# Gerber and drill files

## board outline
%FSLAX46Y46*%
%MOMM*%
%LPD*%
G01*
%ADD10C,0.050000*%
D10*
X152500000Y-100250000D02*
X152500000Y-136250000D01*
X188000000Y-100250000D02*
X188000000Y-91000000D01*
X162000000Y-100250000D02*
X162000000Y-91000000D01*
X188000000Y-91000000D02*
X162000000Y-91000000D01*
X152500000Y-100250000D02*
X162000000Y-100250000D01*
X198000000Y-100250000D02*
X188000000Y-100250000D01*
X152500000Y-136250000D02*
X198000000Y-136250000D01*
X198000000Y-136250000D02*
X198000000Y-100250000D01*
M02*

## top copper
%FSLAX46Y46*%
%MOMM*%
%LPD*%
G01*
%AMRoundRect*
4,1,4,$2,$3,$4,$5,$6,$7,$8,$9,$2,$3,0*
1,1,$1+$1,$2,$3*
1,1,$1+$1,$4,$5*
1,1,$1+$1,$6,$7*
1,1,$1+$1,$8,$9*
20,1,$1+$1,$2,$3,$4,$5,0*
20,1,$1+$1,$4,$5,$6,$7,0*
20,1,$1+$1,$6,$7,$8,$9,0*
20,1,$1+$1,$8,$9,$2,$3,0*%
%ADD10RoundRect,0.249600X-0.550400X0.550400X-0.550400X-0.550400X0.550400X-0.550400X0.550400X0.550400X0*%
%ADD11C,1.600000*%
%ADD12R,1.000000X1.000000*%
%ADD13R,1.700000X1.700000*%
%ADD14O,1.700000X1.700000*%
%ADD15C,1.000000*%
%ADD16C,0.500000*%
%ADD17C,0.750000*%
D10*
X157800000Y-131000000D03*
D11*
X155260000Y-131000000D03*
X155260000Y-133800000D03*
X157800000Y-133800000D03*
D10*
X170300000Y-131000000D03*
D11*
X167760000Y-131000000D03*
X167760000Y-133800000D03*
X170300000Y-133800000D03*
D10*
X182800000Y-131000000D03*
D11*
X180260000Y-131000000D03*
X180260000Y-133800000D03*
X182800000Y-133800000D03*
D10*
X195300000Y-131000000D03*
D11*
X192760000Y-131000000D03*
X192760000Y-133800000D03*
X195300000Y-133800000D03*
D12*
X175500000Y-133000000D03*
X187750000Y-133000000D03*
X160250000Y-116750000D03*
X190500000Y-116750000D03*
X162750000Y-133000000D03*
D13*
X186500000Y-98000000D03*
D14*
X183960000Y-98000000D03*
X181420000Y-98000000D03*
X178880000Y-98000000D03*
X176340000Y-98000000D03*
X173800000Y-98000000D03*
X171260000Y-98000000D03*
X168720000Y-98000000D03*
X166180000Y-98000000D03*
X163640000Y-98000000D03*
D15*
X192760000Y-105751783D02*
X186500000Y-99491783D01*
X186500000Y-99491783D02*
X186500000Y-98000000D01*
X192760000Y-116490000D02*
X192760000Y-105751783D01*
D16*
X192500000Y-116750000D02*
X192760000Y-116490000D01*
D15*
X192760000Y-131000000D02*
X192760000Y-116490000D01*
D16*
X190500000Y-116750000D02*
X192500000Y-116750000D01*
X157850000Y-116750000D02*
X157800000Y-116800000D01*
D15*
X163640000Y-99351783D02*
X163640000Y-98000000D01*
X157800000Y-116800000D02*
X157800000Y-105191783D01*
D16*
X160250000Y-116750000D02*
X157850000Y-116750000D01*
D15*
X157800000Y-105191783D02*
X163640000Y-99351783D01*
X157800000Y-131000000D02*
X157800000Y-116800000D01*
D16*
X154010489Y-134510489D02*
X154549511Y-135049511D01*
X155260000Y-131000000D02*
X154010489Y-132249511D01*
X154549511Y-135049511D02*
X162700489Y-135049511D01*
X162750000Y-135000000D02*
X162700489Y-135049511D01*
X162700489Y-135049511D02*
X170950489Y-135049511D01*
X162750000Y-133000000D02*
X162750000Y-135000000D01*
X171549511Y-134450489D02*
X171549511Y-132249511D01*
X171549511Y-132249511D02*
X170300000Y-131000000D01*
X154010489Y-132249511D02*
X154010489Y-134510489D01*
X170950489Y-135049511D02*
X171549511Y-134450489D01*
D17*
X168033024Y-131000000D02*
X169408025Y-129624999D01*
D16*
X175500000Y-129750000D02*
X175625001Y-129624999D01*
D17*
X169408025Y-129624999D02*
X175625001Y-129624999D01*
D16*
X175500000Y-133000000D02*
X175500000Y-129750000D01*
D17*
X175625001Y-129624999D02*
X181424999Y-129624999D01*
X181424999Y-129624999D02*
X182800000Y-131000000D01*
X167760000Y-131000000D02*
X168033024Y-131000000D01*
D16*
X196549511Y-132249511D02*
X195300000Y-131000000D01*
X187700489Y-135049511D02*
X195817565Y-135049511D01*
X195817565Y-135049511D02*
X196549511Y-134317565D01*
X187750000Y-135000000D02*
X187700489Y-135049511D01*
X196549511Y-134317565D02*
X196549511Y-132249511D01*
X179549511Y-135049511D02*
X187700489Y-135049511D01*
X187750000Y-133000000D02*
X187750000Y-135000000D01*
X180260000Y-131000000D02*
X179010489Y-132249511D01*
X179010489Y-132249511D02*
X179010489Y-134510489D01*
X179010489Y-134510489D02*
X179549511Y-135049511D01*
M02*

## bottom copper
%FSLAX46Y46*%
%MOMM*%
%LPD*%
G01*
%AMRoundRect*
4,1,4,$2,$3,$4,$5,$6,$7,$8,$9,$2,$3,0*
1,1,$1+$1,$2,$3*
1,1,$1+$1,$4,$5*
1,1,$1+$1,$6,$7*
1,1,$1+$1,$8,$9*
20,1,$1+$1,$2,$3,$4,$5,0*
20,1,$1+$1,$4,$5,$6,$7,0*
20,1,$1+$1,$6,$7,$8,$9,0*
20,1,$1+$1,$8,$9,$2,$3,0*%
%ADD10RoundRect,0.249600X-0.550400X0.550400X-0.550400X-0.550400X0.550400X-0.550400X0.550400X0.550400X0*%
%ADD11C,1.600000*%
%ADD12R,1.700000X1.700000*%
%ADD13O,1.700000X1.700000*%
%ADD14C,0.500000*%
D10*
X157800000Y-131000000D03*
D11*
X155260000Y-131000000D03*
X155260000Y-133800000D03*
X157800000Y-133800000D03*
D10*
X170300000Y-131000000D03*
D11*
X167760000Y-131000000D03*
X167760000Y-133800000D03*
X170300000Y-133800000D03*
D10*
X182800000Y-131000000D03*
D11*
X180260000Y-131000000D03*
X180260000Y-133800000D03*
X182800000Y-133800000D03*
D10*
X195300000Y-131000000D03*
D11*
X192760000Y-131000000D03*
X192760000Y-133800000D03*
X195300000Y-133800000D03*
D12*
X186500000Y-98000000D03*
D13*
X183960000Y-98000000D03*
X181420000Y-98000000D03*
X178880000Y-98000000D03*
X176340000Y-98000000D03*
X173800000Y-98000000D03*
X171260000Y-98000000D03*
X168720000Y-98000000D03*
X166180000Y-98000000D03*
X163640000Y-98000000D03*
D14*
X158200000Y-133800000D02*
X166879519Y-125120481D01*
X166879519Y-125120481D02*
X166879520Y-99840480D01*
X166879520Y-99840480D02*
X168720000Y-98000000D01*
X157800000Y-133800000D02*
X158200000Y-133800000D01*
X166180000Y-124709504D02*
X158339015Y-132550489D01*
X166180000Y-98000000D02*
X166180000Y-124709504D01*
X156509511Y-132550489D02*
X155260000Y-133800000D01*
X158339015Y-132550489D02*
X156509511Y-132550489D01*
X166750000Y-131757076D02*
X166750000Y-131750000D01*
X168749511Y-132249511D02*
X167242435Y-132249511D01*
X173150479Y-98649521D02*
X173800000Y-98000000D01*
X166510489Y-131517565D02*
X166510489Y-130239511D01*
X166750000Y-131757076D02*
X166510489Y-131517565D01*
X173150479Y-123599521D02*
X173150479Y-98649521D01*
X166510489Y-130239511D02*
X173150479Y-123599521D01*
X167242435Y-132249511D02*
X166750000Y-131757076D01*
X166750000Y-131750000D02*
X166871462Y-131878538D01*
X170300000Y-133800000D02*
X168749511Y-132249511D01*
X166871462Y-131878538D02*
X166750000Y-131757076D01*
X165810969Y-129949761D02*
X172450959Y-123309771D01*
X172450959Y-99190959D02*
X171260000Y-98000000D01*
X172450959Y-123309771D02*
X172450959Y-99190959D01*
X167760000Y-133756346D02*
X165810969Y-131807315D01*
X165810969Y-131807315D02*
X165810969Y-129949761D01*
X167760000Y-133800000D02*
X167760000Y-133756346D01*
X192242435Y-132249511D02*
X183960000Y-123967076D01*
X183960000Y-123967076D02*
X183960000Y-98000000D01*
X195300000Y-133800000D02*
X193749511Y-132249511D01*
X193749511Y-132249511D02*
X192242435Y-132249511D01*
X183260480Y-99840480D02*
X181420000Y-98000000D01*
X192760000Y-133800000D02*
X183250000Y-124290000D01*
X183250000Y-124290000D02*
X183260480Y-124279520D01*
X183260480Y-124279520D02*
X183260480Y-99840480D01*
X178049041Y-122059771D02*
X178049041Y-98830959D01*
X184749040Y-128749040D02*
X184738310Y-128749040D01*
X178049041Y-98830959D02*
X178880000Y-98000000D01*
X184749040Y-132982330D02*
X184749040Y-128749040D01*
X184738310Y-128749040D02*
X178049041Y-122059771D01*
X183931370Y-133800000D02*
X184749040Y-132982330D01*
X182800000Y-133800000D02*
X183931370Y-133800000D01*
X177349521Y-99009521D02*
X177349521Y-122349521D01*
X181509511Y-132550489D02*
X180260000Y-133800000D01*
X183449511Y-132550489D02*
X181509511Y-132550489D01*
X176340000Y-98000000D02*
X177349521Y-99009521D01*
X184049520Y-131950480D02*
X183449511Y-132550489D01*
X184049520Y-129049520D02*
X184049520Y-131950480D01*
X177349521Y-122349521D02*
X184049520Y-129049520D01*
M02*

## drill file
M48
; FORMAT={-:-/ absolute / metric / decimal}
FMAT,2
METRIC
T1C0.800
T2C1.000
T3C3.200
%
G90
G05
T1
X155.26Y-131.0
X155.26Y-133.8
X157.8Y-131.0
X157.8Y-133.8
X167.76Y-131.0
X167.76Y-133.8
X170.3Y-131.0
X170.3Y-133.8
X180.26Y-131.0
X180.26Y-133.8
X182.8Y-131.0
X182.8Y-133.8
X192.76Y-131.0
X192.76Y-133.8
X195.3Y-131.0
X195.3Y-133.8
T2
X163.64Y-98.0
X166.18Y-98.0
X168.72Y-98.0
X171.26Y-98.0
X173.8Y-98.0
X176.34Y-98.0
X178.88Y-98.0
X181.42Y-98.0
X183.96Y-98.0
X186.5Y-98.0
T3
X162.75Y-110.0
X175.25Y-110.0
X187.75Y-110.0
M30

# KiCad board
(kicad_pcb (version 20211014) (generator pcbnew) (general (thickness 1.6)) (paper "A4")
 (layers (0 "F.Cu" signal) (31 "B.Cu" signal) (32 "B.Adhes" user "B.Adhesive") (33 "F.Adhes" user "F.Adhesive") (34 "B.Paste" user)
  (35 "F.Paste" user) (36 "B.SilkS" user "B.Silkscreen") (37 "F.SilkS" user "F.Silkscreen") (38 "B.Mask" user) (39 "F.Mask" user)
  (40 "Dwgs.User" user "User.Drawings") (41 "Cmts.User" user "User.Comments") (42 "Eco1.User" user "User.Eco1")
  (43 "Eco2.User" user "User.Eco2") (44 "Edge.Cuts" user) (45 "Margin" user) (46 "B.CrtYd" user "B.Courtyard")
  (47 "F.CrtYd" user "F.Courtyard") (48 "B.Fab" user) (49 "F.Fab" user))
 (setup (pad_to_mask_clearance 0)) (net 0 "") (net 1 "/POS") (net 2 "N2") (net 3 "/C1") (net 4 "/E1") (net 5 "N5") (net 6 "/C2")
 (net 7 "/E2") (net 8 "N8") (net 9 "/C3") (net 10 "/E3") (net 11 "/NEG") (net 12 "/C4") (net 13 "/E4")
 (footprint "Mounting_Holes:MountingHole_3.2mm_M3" (layer "F.Cu") (at 162.75 110)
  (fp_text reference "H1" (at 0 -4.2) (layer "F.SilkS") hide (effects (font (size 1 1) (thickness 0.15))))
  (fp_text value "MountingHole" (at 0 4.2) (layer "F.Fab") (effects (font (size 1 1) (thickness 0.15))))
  (pad "" np_thru_hole circle locked (at 0 0) (size 3.2 3.2) (drill 3.2) (layers *.Cu *.Mask)))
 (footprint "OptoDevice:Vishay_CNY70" (layer "F.Cu") (at 157.8 131 -90)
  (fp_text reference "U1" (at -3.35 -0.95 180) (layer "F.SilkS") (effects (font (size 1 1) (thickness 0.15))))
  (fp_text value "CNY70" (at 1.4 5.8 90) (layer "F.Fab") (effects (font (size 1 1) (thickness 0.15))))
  (pad "1" thru_hole roundrect (at 0 0 270) (size 1.6 1.6) (drill 0.8) (layers *.Cu *.Mask) (roundrect_rratio 0.156) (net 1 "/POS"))
  (pad "2" thru_hole circle (at 0 2.54 270) (size 1.6 1.6) (drill 0.8) (layers *.Cu *.Mask) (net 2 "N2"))
  (pad "3" thru_hole circle (at 2.8 2.54 270) (size 1.6 1.6) (drill 0.8) (layers *.Cu *.Mask) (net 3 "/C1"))
  (pad "4" thru_hole circle (at 2.8 0 270) (size 1.6 1.6) (drill 0.8) (layers *.Cu *.Mask) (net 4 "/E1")))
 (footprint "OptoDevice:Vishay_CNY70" (layer "F.Cu") (at 170.3 131 -90)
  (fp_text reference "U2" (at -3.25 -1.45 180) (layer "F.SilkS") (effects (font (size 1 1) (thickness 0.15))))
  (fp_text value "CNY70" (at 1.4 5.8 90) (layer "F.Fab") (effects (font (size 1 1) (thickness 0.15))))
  (pad "1" thru_hole roundrect (at 0 0 270) (size 1.6 1.6) (drill 0.8) (layers *.Cu *.Mask) (roundrect_rratio 0.156) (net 2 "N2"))
  (pad "2" thru_hole circle (at 0 2.54 270) (size 1.6 1.6) (drill 0.8) (layers *.Cu *.Mask) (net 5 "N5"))
  (pad "3" thru_hole circle (at 2.8 2.54 270) (size 1.6 1.6) (drill 0.8) (layers *.Cu *.Mask) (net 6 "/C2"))
  (pad "4" thru_hole circle (at 2.8 0 270) (size 1.6 1.6) (drill 0.8) (layers *.Cu *.Mask) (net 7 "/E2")))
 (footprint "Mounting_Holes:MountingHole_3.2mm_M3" (layer "F.Cu") (at 175.25 110)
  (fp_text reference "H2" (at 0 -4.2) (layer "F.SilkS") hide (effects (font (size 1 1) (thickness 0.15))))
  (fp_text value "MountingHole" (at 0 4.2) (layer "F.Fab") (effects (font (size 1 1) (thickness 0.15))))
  (pad "" np_thru_hole circle locked (at 0 0) (size 3.2 3.2) (drill 3.2) (layers *.Cu *.Mask)))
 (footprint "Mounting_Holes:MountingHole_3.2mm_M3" (layer "F.Cu") (at 187.75 110)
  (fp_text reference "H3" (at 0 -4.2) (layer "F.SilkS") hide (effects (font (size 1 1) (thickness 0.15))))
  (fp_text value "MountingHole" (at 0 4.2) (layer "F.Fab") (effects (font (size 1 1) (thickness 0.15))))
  (pad "" np_thru_hole circle locked (at 0 0) (size 3.2 3.2) (drill 3.2) (layers *.Cu *.Mask)))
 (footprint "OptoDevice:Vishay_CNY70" (layer "F.Cu") (at 182.8 131 -90)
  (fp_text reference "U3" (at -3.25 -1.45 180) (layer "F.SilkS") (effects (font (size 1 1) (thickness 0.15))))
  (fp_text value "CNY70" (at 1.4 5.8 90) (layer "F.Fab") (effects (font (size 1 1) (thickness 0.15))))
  (pad "1" thru_hole roundrect (at 0 0 270) (size 1.6 1.6) (drill 0.8) (layers *.Cu *.Mask) (roundrect_rratio 0.156) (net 5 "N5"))
  (pad "2" thru_hole circle (at 0 2.54 270) (size 1.6 1.6) (drill 0.8) (layers *.Cu *.Mask) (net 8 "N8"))
  (pad "3" thru_hole circle (at 2.8 2.54 270) (size 1.6 1.6) (drill 0.8) (layers *.Cu *.Mask) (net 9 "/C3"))
  (pad "4" thru_hole circle (at 2.8 0 270) (size 1.6 1.6) (drill 0.8) (layers *.Cu *.Mask) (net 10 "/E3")))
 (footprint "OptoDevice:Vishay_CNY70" (layer "F.Cu") (at 195.3 131 -90)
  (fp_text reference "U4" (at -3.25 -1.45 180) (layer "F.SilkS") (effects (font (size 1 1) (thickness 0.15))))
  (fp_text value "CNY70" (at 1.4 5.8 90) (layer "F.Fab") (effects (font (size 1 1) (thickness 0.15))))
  (pad "1" thru_hole roundrect (at 0 0 270) (size 1.6 1.6) (drill 0.8) (layers *.Cu *.Mask) (roundrect_rratio 0.156) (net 8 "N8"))
  (pad "2" thru_hole circle (at 0 2.54 270) (size 1.6 1.6) (drill 0.8) (layers *.Cu *.Mask) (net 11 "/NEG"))
  (pad "3" thru_hole circle (at 2.8 2.54 270) (size 1.6 1.6) (drill 0.8) (layers *.Cu *.Mask) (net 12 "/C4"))
  (pad "4" thru_hole circle (at 2.8 0 270) (size 1.6 1.6) (drill 0.8) (layers *.Cu *.Mask) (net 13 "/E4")))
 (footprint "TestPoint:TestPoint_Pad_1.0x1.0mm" (layer "F.Cu") (at 175.5 133)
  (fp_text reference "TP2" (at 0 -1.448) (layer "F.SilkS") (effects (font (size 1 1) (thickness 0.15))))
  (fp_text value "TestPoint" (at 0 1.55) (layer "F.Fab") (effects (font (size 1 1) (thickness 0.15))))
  (pad "1" smd rect locked (at 0 0) (size 1 1) (layers "F.Cu" "F.Mask") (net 5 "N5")))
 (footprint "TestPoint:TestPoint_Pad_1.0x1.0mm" (layer "F.Cu") (at 187.75 133)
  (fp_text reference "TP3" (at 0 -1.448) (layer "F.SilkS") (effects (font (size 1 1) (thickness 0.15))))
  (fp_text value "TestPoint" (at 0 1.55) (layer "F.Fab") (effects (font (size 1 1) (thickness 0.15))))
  (pad "1" smd rect locked (at 0 0) (size 1 1) (layers "F.Cu" "F.Mask") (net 8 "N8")))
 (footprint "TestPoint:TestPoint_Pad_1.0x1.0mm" (layer "F.Cu") (at 160.25 116.75)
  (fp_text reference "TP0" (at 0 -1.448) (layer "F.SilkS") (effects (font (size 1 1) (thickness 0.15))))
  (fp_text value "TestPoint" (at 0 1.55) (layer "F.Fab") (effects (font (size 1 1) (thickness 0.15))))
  (pad "1" smd rect locked (at 0 0) (size 1 1) (layers "F.Cu" "F.Mask") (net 1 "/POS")))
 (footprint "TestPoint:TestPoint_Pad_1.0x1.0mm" (layer "F.Cu") (at 190.5 116.75)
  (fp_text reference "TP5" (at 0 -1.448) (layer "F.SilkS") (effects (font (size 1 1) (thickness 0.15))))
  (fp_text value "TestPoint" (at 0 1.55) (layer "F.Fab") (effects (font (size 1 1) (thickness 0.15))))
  (pad "1" smd rect locked (at 0 0) (size 1 1) (layers "F.Cu" "F.Mask") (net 11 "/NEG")))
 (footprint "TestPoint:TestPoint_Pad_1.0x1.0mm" (layer "F.Cu") (at 162.75 133)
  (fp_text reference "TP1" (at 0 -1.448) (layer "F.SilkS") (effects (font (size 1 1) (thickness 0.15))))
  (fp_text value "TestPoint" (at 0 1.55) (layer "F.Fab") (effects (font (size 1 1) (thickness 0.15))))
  (pad "1" smd rect locked (at 0 0) (size 1 1) (layers "F.Cu" "F.Mask") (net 2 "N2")))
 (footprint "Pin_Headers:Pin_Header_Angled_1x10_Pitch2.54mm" (layer "B.Cu") (at 186.5 98 90)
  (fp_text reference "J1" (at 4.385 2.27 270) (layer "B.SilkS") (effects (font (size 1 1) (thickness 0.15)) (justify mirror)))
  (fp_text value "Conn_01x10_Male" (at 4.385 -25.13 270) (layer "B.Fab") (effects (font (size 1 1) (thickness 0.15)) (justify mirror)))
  (pad "1" thru_hole rect (at 0 0 90) (size 1.7 1.7) (drill 1) (layers *.Cu *.Mask) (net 11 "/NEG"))
  (pad "2" thru_hole oval (at 0 -2.54 90) (size 1.7 1.7) (drill 1) (layers *.Cu *.Mask) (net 13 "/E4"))
  (pad "3" thru_hole oval (at 0 -5.08 90) (size 1.7 1.7) (drill 1) (layers *.Cu *.Mask) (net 12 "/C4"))
  (pad "4" thru_hole oval (at 0 -7.62 90) (size 1.7 1.7) (drill 1) (layers *.Cu *.Mask) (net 10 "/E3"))
  (pad "5" thru_hole oval (at 0 -10.16 90) (size 1.7 1.7) (drill 1) (layers *.Cu *.Mask) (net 9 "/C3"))
  (pad "6" thru_hole oval (at 0 -12.7 90) (size 1.7 1.7) (drill 1) (layers *.Cu *.Mask) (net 7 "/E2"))
  (pad "7" thru_hole oval (at 0 -15.24 90) (size 1.7 1.7) (drill 1) (layers *.Cu *.Mask) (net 6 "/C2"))
  (pad "8" thru_hole oval (at 0 -17.78 90) (size 1.7 1.7) (drill 1) (layers *.Cu *.Mask) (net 4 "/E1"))
  (pad "9" thru_hole oval (at 0 -20.32 90) (size 1.7 1.7) (drill 1) (layers *.Cu *.Mask) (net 3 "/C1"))
  (pad "10" thru_hole oval (at 0 -22.86 90) (size 1.7 1.7) (drill 1) (layers *.Cu *.Mask) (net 1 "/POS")))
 (gr_line (start 152.5 100.25) (end 152.5 136.25) (layer "Edge.Cuts") (width 0.05))
 (gr_line (start 188 100.25) (end 188 91) (layer "Edge.Cuts") (width 0.05))
 (gr_line (start 162 100.25) (end 162 91) (layer "Edge.Cuts") (width 0.05))
 (gr_line (start 188 91) (end 162 91) (layer "Edge.Cuts") (width 0.05))
 (gr_line (start 152.5 100.25) (end 162 100.25) (layer "Edge.Cuts") (width 0.05))
 (gr_line (start 198 100.25) (end 188 100.25) (layer "Edge.Cuts") (width 0.05))
 (gr_line (start 152.5 136.25) (end 198 136.25) (layer "Edge.Cuts") (width 0.05))
 (gr_line (start 198 136.25) (end 198 100.25) (layer "Edge.Cuts") (width 0.05))
 (segment (start 192.76 105.751783) (end 186.5 99.491783) (width 1) (layer "F.Cu") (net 11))
 (segment (start 186.5 99.491783) (end 186.5 98) (width 1) (layer "F.Cu") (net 11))
 (segment (start 192.76 116.49) (end 192.76 105.751783) (width 1) (layer "F.Cu") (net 11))
 (segment (start 192.5 116.75) (end 192.76 116.49) (width 0.5) (layer "F.Cu") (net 11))
 (segment (start 192.76 131) (end 192.76 116.49) (width 1) (layer "F.Cu") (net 11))
 (segment (start 190.5 116.75) (end 192.5 116.75) (width 0.5) (layer "F.Cu") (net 11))
 (segment (start 158.2 133.8) (end 166.879519 125.120481) (width 0.5) (layer "B.Cu") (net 4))
 (segment (start 166.879519 125.120481) (end 166.87952 99.84048) (width 0.5) (layer "B.Cu") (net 4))
 (segment (start 166.87952 99.84048) (end 168.72 98) (width 0.5) (layer "B.Cu") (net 4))
 (segment (start 157.8 133.8) (end 158.2 133.8) (width 0.5) (layer "B.Cu") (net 4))
 (segment (start 166.18 124.709504) (end 158.339015 132.550489) (width 0.5) (layer "B.Cu") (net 3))
 (segment (start 166.18 98) (end 166.18 124.709504) (width 0.5) (layer "B.Cu") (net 3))
 (segment (start 156.509511 132.550489) (end 155.26 133.8) (width 0.5) (layer "B.Cu") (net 3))
 (segment (start 158.339015 132.550489) (end 156.509511 132.550489) (width 0.5) (layer "B.Cu") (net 3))
 (segment (start 157.85 116.75) (end 157.8 116.8) (width 0.5) (layer "F.Cu") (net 1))
 (segment (start 163.64 99.351783) (end 163.64 98) (width 1) (layer "F.Cu") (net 1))
 (segment (start 157.8 116.8) (end 157.8 105.191783) (width 1) (layer "F.Cu") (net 1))
 (segment (start 160.25 116.75) (end 157.85 116.75) (width 0.5) (layer "F.Cu") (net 1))
 (segment (start 157.8 105.191783) (end 163.64 99.351783) (width 1) (layer "F.Cu") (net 1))
 (segment (start 157.8 131) (end 157.8 116.8) (width 1) (layer "F.Cu") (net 1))
 (segment (start 154.010489 134.510489) (end 154.549511 135.049511) (width 0.5) (layer "F.Cu") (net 2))
 (segment (start 155.26 131) (end 154.010489 132.249511) (width 0.5) (layer "F.Cu") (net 2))
 (segment (start 154.549511 135.049511) (end 162.700489 135.049511) (width 0.5) (layer "F.Cu") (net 2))
 (segment (start 162.75 135) (end 162.700489 135.049511) (width 0.5) (layer "F.Cu") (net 2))
 (segment (start 162.700489 135.049511) (end 170.950489 135.049511) (width 0.5) (layer "F.Cu") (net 2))
 (segment (start 162.75 133) (end 162.75 135) (width 0.5) (layer "F.Cu") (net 2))
 (segment (start 171.549511 134.450489) (end 171.549511 132.249511) (width 0.5) (layer "F.Cu") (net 2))
 (segment (start 171.549511 132.249511) (end 170.3 131) (width 0.5) (layer "F.Cu") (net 2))
 (segment (start 154.010489 132.249511) (end 154.010489 134.510489) (width 0.5) (layer "F.Cu") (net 2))
 (segment (start 170.950489 135.049511) (end 171.549511 134.450489) (width 0.5) (layer "F.Cu") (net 2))
 (segment (start 166.75 131.757076) (end 166.75 131.75) (width 0.5) (layer "B.Cu") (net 7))
 (segment (start 168.749511 132.249511) (end 167.242435 132.249511) (width 0.5) (layer "B.Cu") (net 7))
 (segment (start 173.150479 98.649521) (end 173.8 98) (width 0.5) (layer "B.Cu") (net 7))
 (segment (start 166.510489 131.517565) (end 166.510489 130.239511) (width 0.5) (layer "B.Cu") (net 7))
 (segment (start 166.75 131.757076) (end 166.510489 131.517565) (width 0.5) (layer "B.Cu") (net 7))
 (segment (start 173.150479 123.599521) (end 173.150479 98.649521) (width 0.5) (layer "B.Cu") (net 7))
 (segment (start 166.510489 130.239511) (end 173.150479 123.599521) (width 0.5) (layer "B.Cu") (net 7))
 (segment (start 167.242435 132.249511) (end 166.75 131.757076) (width 0.5) (layer "B.Cu") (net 7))
 (segment (start 166.75 131.75) (end 166.871462 131.878538) (width 0.5) (layer "B.Cu") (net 7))
 (segment (start 170.3 133.8) (end 168.749511 132.249511) (width 0.5) (layer "B.Cu") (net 7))
 (segment (start 166.871462 131.878538) (end 166.75 131.757076) (width 0.5) (layer "B.Cu") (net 7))
 (segment (start 165.810969 129.949761) (end 172.450959 123.309771) (width 0.5) (layer "B.Cu") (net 6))
 (segment (start 172.450959 99.190959) (end 171.26 98) (width 0.5) (layer "B.Cu") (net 6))
 (segment (start 172.450959 123.309771) (end 172.450959 99.190959) (width 0.5) (layer "B.Cu") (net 6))
 (segment (start 167.76 133.756346) (end 165.810969 131.807315) (width 0.5) (layer "B.Cu") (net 6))
 (segment (start 165.810969 131.807315) (end 165.810969 129.949761) (width 0.5) (layer "B.Cu") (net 6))
 (segment (start 167.76 133.8) (end 167.76 133.756346) (width 0.5) (layer "B.Cu") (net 6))
 (segment (start 192.242435 132.249511) (end 183.96 123.967076) (width 0.5) (layer "B.Cu") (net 13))
 (segment (start 183.96 123.967076) (end 183.96 98) (width 0.5) (layer "B.Cu") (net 13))
 (segment (start 195.3 133.8) (end 193.749511 132.249511) (width 0.5) (layer "B.Cu") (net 13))
 (segment (start 193.749511 132.249511) (end 192.242435 132.249511) (width 0.5) (layer "B.Cu") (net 13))
 (segment (start 183.26048 99.84048) (end 181.42 98) (width 0.5) (layer "B.Cu") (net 12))
 (segment (start 192.76 133.8) (end 183.25 124.29) (width 0.5) (layer "B.Cu") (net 12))
 (segment (start 183.25 124.29) (end 183.26048 124.27952) (width 0.5) (layer "B.Cu") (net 12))
 (segment (start 183.26048 124.27952) (end 183.26048 99.84048) (width 0.5) (layer "B.Cu") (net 12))
 (segment (start 178.049041 122.059771) (end 178.049041 98.830959) (width 0.5) (layer "B.Cu") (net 10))
 (segment (start 184.74904 128.74904) (end 184.73831 128.74904) (width 0.5) (layer "B.Cu") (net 10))
 (segment (start 178.049041 98.830959) (end 178.88 98) (width 0.5) (layer "B.Cu") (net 10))
 (segment (start 184.74904 132.98233) (end 184.74904 128.74904) (width 0.5) (layer "B.Cu") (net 10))
 (segment (start 184.73831 128.74904) (end 178.049041 122.059771) (width 0.5) (layer "B.Cu") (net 10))
 (segment (start 183.93137 133.8) (end 184.74904 132.98233) (width 0.5) (layer "B.Cu") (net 10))
 (segment (start 182.8 133.8) (end 183.93137 133.8) (width 0.5) (layer "B.Cu") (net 10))
 (segment (start 177.349521 99.009521) (end 177.349521 122.349521) (width 0.5) (layer "B.Cu") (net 9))
 (segment (start 181.509511 132.550489) (end 180.26 133.8) (width 0.5) (layer "B.Cu") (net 9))
 (segment (start 183.449511 132.550489) (end 181.509511 132.550489) (width 0.5) (layer "B.Cu") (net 9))
 (segment (start 176.34 98) (end 177.349521 99.009521) (width 0.5) (layer "B.Cu") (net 9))
 (segment (start 184.04952 131.95048) (end 183.449511 132.550489) (width 0.5) (layer "B.Cu") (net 9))
 (segment (start 184.04952 129.04952) (end 184.04952 131.95048) (width 0.5) (layer "B.Cu") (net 9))
 (segment (start 177.349521 122.349521) (end 184.04952 129.04952) (width 0.5) (layer "B.Cu") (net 9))
 (segment (start 168.033024 131) (end 169.408025 129.624999) (width 0.75) (layer "F.Cu") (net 5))
 (segment (start 175.5 129.75) (end 175.625001 129.624999) (width 0.5) (layer "F.Cu") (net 5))
 (segment (start 169.408025 129.624999) (end 175.625001 129.624999) (width 0.75) (layer "F.Cu") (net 5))
 (segment (start 175.5 133) (end 175.5 129.75) (width 0.5) (layer "F.Cu") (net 5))
 (segment (start 175.625001 129.624999) (end 181.424999 129.624999) (width 0.75) (layer "F.Cu") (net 5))
 (segment (start 181.424999 129.624999) (end 182.8 131) (width 0.75) (layer "F.Cu") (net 5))
 (segment (start 167.76 131) (end 168.033024 131) (width 0.75) (layer "F.Cu") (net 5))
 (segment (start 196.549511 132.249511) (end 195.3 131) (width 0.5) (layer "F.Cu") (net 8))
 (segment (start 187.700489 135.049511) (end 195.817565 135.049511) (width 0.5) (layer "F.Cu") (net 8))
 (segment (start 195.817565 135.049511) (end 196.549511 134.317565) (width 0.5) (layer "F.Cu") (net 8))
 (segment (start 187.75 135) (end 187.700489 135.049511) (width 0.5) (layer "F.Cu") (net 8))
 (segment (start 196.549511 134.317565) (end 196.549511 132.249511) (width 0.5) (layer "F.Cu") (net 8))
 (segment (start 179.549511 135.049511) (end 187.700489 135.049511) (width 0.5) (layer "F.Cu") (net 8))
 (segment (start 187.75 133) (end 187.75 135) (width 0.5) (layer "F.Cu") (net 8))
 (segment (start 180.26 131) (end 179.010489 132.249511) (width 0.5) (layer "F.Cu") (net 8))
 (segment (start 179.010489 132.249511) (end 179.010489 134.510489) (width 0.5) (layer "F.Cu") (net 8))
 (segment (start 179.010489 134.510489) (end 179.549511 135.049511) (width 0.5) (layer "F.Cu") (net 8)))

